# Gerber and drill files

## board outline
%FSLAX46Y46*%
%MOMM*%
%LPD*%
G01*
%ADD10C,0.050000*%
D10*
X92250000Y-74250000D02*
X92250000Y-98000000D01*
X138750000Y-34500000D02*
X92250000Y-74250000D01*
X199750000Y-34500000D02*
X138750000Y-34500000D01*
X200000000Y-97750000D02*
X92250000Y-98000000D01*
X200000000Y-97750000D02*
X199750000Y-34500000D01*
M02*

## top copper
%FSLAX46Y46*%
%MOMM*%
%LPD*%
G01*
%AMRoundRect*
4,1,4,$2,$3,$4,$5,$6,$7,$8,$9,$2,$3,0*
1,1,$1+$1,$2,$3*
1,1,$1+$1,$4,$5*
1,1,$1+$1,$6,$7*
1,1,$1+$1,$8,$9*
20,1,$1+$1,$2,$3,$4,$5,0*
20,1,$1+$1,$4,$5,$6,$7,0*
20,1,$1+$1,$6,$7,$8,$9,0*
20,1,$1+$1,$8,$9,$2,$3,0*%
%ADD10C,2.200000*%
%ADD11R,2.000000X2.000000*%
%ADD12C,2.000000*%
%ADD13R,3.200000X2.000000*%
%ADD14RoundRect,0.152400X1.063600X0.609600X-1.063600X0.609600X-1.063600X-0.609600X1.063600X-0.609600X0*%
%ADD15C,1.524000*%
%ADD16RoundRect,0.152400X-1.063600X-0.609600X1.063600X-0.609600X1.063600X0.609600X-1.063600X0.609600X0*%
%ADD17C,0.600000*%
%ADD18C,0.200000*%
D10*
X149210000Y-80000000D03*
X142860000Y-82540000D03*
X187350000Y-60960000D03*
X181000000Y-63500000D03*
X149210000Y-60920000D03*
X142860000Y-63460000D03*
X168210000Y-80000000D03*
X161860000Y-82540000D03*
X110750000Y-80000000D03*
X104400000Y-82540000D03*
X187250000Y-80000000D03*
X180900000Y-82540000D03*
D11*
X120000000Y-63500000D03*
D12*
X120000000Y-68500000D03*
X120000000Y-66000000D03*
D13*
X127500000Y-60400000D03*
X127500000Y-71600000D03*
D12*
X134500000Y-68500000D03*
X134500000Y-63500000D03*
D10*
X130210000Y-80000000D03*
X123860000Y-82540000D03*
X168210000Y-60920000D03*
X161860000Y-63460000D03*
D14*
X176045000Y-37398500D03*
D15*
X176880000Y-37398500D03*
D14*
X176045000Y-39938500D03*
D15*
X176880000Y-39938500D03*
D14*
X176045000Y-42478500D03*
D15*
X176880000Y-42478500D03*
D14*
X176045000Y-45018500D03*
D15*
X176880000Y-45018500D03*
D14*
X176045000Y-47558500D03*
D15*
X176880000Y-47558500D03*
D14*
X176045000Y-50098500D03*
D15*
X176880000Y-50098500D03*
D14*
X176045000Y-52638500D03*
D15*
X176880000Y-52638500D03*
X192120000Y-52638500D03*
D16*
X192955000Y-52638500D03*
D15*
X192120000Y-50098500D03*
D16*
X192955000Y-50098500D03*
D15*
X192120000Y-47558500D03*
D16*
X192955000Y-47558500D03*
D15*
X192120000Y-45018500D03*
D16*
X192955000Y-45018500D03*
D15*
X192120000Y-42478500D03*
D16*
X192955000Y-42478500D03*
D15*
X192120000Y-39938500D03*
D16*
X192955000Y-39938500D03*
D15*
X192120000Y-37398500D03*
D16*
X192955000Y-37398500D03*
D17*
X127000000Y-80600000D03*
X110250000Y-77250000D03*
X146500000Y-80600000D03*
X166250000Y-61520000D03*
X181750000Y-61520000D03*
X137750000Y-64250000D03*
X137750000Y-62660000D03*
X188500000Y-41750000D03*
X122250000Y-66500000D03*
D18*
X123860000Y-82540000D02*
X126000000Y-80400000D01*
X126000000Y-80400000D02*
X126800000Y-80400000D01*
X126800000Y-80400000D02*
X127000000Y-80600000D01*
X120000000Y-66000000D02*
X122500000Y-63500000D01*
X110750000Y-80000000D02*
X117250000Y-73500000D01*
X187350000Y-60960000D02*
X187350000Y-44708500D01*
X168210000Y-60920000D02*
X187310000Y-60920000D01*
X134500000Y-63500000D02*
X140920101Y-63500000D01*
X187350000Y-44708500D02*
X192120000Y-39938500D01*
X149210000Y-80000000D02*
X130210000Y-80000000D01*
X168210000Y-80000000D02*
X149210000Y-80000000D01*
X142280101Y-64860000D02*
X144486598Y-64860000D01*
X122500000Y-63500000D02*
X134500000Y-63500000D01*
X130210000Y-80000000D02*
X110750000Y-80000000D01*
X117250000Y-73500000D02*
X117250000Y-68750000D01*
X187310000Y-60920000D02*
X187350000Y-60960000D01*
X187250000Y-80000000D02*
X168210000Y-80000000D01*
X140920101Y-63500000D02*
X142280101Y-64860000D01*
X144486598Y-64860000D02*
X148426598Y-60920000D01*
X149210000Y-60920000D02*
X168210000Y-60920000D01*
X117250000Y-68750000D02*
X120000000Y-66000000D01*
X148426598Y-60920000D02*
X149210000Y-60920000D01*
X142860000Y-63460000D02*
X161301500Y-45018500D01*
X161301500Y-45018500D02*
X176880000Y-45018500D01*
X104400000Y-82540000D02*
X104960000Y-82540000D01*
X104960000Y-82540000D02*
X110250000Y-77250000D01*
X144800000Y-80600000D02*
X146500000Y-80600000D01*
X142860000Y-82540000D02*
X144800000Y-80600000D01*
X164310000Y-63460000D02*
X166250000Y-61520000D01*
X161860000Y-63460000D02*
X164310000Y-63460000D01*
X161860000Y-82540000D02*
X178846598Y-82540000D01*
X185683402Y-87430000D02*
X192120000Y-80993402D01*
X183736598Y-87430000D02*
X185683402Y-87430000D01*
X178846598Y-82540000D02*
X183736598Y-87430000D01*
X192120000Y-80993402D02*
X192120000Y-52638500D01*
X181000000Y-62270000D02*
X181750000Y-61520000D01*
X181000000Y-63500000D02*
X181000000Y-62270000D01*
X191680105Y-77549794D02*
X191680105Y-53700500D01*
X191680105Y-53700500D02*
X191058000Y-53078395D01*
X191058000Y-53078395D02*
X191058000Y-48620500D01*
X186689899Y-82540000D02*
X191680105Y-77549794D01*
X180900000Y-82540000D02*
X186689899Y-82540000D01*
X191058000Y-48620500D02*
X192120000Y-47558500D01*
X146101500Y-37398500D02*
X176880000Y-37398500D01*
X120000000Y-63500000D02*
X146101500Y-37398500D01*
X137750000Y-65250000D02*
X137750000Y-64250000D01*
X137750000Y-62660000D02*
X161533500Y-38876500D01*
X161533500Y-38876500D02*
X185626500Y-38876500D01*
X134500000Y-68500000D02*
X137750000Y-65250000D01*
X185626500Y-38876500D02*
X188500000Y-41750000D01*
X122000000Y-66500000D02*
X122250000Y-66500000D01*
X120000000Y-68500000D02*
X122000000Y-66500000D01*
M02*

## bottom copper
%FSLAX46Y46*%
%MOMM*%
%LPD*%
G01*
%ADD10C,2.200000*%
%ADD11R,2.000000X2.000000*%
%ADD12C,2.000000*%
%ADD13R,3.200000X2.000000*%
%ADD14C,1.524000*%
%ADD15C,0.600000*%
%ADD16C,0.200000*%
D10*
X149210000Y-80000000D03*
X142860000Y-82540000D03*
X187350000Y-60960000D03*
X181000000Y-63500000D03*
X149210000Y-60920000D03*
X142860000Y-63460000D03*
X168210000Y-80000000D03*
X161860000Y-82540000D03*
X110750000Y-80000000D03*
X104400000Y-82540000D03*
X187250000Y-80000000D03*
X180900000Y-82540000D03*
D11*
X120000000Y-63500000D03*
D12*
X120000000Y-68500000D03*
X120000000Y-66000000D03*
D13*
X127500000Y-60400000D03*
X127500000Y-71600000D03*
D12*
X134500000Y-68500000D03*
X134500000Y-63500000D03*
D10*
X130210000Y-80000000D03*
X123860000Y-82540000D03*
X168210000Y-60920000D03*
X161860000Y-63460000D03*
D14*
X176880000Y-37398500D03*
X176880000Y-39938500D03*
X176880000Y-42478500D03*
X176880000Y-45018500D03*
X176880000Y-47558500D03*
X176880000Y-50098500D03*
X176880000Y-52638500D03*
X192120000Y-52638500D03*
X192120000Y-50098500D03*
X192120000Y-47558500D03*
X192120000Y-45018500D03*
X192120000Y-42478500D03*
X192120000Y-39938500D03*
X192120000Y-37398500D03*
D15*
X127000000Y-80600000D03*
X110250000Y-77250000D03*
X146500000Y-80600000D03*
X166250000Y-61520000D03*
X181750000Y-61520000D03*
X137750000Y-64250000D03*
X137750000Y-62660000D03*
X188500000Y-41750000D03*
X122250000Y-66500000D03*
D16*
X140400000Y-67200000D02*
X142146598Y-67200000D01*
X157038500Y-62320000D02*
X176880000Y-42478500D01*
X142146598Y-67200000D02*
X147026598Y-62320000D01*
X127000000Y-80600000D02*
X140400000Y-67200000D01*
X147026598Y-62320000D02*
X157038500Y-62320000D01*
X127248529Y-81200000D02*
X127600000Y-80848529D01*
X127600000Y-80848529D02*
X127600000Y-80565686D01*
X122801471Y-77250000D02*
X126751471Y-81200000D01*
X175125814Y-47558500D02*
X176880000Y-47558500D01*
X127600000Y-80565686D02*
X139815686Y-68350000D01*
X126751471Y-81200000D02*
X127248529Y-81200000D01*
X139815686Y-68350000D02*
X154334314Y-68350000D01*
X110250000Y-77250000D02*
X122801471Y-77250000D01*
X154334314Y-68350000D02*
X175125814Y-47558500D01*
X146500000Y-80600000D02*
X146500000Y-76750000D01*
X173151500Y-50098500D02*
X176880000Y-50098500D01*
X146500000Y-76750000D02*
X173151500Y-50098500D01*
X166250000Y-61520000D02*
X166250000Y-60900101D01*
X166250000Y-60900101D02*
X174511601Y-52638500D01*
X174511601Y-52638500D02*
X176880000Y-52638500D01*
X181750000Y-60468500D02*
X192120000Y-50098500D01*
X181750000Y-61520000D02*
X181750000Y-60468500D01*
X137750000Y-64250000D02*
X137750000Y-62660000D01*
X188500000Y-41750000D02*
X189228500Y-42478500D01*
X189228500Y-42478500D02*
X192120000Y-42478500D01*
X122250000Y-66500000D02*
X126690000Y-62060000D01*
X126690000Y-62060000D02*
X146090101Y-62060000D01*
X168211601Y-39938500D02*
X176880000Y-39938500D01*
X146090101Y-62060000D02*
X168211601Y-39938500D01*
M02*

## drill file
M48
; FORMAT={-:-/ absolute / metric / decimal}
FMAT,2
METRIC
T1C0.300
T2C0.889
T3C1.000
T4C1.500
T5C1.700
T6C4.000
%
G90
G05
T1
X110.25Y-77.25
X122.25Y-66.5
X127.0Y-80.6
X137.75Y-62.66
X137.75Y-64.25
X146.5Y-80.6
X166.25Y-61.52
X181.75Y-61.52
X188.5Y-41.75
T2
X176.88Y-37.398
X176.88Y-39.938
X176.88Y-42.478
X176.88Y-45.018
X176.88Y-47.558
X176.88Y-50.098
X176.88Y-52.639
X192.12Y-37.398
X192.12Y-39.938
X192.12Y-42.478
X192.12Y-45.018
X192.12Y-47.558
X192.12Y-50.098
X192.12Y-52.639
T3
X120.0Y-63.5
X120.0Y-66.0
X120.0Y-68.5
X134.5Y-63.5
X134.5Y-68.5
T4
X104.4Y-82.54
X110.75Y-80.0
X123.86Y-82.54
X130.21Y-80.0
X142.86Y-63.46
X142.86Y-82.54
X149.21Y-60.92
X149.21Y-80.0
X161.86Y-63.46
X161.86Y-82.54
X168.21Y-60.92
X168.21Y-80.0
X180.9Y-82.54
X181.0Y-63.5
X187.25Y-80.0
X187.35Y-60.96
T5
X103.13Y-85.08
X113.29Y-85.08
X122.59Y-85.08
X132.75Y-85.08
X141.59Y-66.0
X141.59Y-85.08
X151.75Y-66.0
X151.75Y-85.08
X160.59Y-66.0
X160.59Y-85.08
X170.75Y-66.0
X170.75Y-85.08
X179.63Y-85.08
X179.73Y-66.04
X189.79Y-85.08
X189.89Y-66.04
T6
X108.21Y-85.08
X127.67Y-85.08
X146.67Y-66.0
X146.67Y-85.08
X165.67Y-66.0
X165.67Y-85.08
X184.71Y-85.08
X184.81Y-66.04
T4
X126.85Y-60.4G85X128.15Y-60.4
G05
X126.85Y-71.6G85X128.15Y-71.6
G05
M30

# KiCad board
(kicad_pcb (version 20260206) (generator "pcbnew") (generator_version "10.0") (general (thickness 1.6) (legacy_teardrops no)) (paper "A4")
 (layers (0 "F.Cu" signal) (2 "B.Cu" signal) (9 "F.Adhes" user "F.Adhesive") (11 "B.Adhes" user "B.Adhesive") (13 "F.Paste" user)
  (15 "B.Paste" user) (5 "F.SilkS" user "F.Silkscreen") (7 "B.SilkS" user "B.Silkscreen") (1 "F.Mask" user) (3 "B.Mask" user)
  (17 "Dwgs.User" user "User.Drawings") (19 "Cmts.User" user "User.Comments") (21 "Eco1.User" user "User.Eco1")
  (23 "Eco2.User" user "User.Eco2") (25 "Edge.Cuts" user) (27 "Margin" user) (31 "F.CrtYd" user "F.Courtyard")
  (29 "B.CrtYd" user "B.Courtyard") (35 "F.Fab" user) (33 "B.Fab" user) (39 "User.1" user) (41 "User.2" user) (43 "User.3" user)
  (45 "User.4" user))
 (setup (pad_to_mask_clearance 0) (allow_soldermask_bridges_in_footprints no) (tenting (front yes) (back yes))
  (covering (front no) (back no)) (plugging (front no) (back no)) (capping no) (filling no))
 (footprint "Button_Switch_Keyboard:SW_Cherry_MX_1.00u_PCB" (layer "F.Cu") (at 149.21 80)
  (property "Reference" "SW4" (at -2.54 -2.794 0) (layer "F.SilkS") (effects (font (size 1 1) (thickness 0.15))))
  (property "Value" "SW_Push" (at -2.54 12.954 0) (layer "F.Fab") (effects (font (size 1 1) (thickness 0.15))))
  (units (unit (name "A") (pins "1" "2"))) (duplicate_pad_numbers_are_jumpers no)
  (pad "" np_thru_hole circle (at -7.62 5.08) (size 1.7 1.7) (drill 1.7) (layers "*.Cu" "*.Mask"))
  (pad "" np_thru_hole circle (at -2.54 5.08) (size 4 4) (drill 4) (layers "*.Cu" "*.Mask"))
  (pad "" np_thru_hole circle (at 2.54 5.08) (size 1.7 1.7) (drill 1.7) (layers "*.Cu" "*.Mask"))
  (pad "1" thru_hole circle (at 0 0) (size 2.2 2.2) (drill 1.5) (layers "*.Cu" "*.Mask") (remove_unused_layers no) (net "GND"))
  (pad "2" thru_hole circle (at -6.35 2.54) (size 2.2 2.2) (drill 1.5) (layers "*.Cu" "*.Mask") (remove_unused_layers no)
   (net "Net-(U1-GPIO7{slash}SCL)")))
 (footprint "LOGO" (layer "F.Cu") (at 117.485008 73.126205 90)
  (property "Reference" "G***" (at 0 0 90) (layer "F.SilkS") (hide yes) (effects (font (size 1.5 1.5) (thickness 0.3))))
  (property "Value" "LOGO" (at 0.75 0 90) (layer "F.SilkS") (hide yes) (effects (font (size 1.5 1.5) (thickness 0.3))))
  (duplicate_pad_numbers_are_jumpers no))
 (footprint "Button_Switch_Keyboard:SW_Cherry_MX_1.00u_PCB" (layer "F.Cu") (at 187.35 60.96)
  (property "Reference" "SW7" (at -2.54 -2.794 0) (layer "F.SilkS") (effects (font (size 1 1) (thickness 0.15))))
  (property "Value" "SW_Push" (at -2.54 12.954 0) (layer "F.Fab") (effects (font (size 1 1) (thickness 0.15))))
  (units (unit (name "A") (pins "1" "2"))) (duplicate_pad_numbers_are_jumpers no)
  (pad "" np_thru_hole circle (at -7.62 5.08) (size 1.7 1.7) (drill 1.7) (layers "*.Cu" "*.Mask"))
  (pad "" np_thru_hole circle (at -2.54 5.08) (size 4 4) (drill 4) (layers "*.Cu" "*.Mask"))
  (pad "" np_thru_hole circle (at 2.54 5.08) (size 1.7 1.7) (drill 1.7) (layers "*.Cu" "*.Mask"))
  (pad "1" thru_hole circle (at 0 0) (size 2.2 2.2) (drill 1.5) (layers "*.Cu" "*.Mask") (remove_unused_layers no) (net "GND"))
  (pad "2" thru_hole circle (at -6.35 2.54) (size 2.2 2.2) (drill 1.5) (layers "*.Cu" "*.Mask") (remove_unused_layers no)
   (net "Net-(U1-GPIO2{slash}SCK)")))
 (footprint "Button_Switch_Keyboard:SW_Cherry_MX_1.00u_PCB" (layer "F.Cu") (at 149.21 60.92)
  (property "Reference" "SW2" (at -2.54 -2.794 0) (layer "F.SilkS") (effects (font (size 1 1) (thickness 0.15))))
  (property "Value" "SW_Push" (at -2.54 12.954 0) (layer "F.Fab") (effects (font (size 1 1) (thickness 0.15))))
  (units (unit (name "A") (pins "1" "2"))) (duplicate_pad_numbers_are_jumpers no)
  (pad "" np_thru_hole circle (at -7.62 5.08) (size 1.7 1.7) (drill 1.7) (layers "*.Cu" "*.Mask"))
  (pad "" np_thru_hole circle (at -2.54 5.08) (size 4 4) (drill 4) (layers "*.Cu" "*.Mask"))
  (pad "" np_thru_hole circle (at 2.54 5.08) (size 1.7 1.7) (drill 1.7) (layers "*.Cu" "*.Mask"))
  (pad "1" thru_hole circle (at 0 0) (size 2.2 2.2) (drill 1.5) (layers "*.Cu" "*.Mask") (remove_unused_layers no) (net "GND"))
  (pad "2" thru_hole circle (at -6.35 2.54) (size 2.2 2.2) (drill 1.5) (layers "*.Cu" "*.Mask") (remove_unused_layers no)
   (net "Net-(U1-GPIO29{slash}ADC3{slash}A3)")))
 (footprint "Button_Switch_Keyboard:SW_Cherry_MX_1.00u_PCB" (layer "F.Cu") (at 168.21 80)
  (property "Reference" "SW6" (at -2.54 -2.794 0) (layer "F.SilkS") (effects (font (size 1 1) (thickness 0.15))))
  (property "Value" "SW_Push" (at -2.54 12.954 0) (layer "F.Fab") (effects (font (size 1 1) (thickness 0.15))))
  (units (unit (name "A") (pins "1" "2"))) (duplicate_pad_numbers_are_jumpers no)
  (pad "" np_thru_hole circle (at -7.62 5.08) (size 1.7 1.7) (drill 1.7) (layers "*.Cu" "*.Mask"))
  (pad "" np_thru_hole circle (at -2.54 5.08) (size 4 4) (drill 4) (layers "*.Cu" "*.Mask"))
  (pad "" np_thru_hole circle (at 2.54 5.08) (size 1.7 1.7) (drill 1.7) (layers "*.Cu" "*.Mask"))
  (pad "1" thru_hole circle (at 0 0) (size 2.2 2.2) (drill 1.5) (layers "*.Cu" "*.Mask") (remove_unused_layers no) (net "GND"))
  (pad "2" thru_hole circle (at -6.35 2.54) (size 2.2 2.2) (drill 1.5) (layers "*.Cu" "*.Mask") (remove_unused_layers no)
   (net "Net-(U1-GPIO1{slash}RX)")))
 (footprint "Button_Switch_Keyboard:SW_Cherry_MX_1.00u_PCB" (layer "F.Cu") (at 110.75 80)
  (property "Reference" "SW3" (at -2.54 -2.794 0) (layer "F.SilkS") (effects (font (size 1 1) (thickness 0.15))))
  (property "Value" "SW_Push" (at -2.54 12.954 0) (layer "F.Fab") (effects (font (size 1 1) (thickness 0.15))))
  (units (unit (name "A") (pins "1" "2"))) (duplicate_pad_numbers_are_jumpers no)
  (pad "" np_thru_hole circle (at -7.62 5.08) (size 1.7 1.7) (drill 1.7) (layers "*.Cu" "*.Mask"))
  (pad "" np_thru_hole circle (at -2.54 5.08) (size 4 4) (drill 4) (layers "*.Cu" "*.Mask"))
  (pad "" np_thru_hole circle (at 2.54 5.08) (size 1.7 1.7) (drill 1.7) (layers "*.Cu" "*.Mask"))
  (pad "1" thru_hole circle (at 0 0) (size 2.2 2.2) (drill 1.5) (layers "*.Cu" "*.Mask") (remove_unused_layers no) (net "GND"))
  (pad "2" thru_hole circle (at -6.35 2.54) (size 2.2 2.2) (drill 1.5) (layers "*.Cu" "*.Mask") (remove_unused_layers no)
   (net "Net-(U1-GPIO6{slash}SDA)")))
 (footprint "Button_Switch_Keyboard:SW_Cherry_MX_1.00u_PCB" (layer "F.Cu") (at 187.25 80)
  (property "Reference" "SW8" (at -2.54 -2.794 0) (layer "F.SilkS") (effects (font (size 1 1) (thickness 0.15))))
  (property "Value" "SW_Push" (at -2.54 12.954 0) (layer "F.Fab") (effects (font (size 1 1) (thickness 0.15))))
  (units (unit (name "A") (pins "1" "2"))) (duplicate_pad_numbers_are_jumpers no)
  (pad "" np_thru_hole circle (at -7.62 5.08) (size 1.7 1.7) (drill 1.7) (layers "*.Cu" "*.Mask"))
  (pad "" np_thru_hole circle (at -2.54 5.08) (size 4 4) (drill 4) (layers "*.Cu" "*.Mask"))
  (pad "" np_thru_hole circle (at 2.54 5.08) (size 1.7 1.7) (drill 1.7) (layers "*.Cu" "*.Mask"))
  (pad "1" thru_hole circle (at 0 0) (size 2.2 2.2) (drill 1.5) (layers "*.Cu" "*.Mask") (remove_unused_layers no) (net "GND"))
  (pad "2" thru_hole circle (at -6.35 2.54) (size 2.2 2.2) (drill 1.5) (layers "*.Cu" "*.Mask") (remove_unused_layers no)
   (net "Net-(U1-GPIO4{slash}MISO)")))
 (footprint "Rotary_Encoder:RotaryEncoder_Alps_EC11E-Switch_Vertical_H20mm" (layer "F.Cu") (at 120 63.5)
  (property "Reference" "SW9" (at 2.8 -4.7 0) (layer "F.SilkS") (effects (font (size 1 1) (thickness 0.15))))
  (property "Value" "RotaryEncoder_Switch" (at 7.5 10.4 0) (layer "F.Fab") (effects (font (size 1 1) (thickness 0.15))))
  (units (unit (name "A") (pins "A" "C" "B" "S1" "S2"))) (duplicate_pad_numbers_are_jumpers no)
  (pad "A" thru_hole rect (at 0 0) (size 2 2) (drill 1) (layers "*.Cu" "*.Mask") (remove_unused_layers no)
   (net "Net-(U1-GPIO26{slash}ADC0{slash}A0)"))
  (pad "B" thru_hole circle (at 0 5) (size 2 2) (drill 1) (layers "*.Cu" "*.Mask") (remove_unused_layers no)
   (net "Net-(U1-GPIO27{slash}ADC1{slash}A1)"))
  (pad "C" thru_hole circle (at 0 2.5) (size 2 2) (drill 1) (layers "*.Cu" "*.Mask") (remove_unused_layers no) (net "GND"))
  (pad "MP" thru_hole rect (at 7.5 -3.1) (size 3.2 2) (drill oval 2.8 1.5) (layers "*.Cu" "*.Mask") (remove_unused_layers no))
  (pad "MP" thru_hole rect (at 7.5 8.1) (size 3.2 2) (drill oval 2.8 1.5) (layers "*.Cu" "*.Mask") (remove_unused_layers no))
  (pad "S1" thru_hole circle (at 14.5 5) (size 2 2) (drill 1) (layers "*.Cu" "*.Mask") (remove_unused_layers no) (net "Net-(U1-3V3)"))
  (pad "S2" thru_hole circle (at 14.5 0) (size 2 2) (drill 1) (layers "*.Cu" "*.Mask") (remove_unused_layers no) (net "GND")))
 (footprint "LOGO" (layer "F.Cu") (at 167.351488 86.633252)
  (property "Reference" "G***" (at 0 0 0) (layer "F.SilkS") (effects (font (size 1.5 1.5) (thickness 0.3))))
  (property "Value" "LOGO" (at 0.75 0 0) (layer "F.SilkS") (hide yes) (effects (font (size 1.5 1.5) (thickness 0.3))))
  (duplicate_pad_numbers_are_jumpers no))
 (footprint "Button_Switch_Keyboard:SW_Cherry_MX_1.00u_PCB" (layer "F.Cu") (at 130.21 80)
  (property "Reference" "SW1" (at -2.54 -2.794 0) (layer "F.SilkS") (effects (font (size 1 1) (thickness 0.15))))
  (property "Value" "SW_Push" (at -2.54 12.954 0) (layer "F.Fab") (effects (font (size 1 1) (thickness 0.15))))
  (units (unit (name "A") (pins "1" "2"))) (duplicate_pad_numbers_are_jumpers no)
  (pad "" np_thru_hole circle (at -7.62 5.08) (size 1.7 1.7) (drill 1.7) (layers "*.Cu" "*.Mask"))
  (pad "" np_thru_hole circle (at -2.54 5.08) (size 4 4) (drill 4) (layers "*.Cu" "*.Mask"))
  (pad "" np_thru_hole circle (at 2.54 5.08) (size 1.7 1.7) (drill 1.7) (layers "*.Cu" "*.Mask"))
  (pad "1" thru_hole circle (at 0 0) (size 2.2 2.2) (drill 1.5) (layers "*.Cu" "*.Mask") (remove_unused_layers no) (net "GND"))
  (pad "2" thru_hole circle (at -6.35 2.54) (size 2.2 2.2) (drill 1.5) (layers "*.Cu" "*.Mask") (remove_unused_layers no)
   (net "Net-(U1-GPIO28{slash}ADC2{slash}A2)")))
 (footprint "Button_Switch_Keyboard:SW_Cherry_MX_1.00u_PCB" (layer "F.Cu") (at 168.21 60.92)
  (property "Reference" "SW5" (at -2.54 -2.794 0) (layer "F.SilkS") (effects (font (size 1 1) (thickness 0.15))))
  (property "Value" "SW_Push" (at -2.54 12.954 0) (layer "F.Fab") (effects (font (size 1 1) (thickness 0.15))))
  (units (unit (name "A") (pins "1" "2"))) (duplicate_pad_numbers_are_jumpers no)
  (pad "" np_thru_hole circle (at -7.62 5.08) (size 1.7 1.7) (drill 1.7) (layers "*.Cu" "*.Mask"))
  (pad "" np_thru_hole circle (at -2.54 5.08) (size 4 4) (drill 4) (layers "*.Cu" "*.Mask"))
  (pad "" np_thru_hole circle (at 2.54 5.08) (size 1.7 1.7) (drill 1.7) (layers "*.Cu" "*.Mask"))
  (pad "1" thru_hole circle (at 0 0) (size 2.2 2.2) (drill 1.5) (layers "*.Cu" "*.Mask") (remove_unused_layers no) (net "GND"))
  (pad "2" thru_hole circle (at -6.35 2.54) (size 2.2 2.2) (drill 1.5) (layers "*.Cu" "*.Mask") (remove_unused_layers no)
   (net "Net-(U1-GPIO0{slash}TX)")))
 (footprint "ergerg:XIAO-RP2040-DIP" (layer "F.Cu") (at 184.5 45.0185)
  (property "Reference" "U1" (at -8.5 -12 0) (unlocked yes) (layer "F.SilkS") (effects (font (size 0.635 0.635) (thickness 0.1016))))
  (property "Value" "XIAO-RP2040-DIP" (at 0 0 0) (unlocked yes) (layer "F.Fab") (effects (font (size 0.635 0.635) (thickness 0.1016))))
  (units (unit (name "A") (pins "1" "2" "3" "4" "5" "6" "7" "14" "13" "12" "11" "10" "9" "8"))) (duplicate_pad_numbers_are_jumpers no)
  (pad "1" smd roundrect (at -8.455 -7.62 180) (size 2.432 1.524) (layers "F.Cu" "F.Mask") (roundrect_rratio 0.1)
   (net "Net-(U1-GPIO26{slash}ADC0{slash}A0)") (thermal_bridge_angle 45))
  (pad "1" thru_hole circle (at -7.62 -7.62 180) (size 1.524 1.524) (drill 0.889) (layers "*.Cu" "*.Mask") (remove_unused_layers no)
   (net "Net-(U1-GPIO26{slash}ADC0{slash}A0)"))
  (pad "2" smd roundrect (at -8.455 -5.08 180) (size 2.432 1.524) (layers "F.Cu" "F.Mask") (roundrect_rratio 0.1)
   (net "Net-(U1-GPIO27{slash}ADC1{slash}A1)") (thermal_bridge_angle 45))
  (pad "2" thru_hole circle (at -7.62 -5.08 180) (size 1.524 1.524) (drill 0.889) (layers "*.Cu" "*.Mask") (remove_unused_layers no)
   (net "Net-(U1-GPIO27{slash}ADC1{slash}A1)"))
  (pad "3" smd roundrect (at -8.455 -2.54 180) (size 2.432 1.524) (layers "F.Cu" "F.Mask") (roundrect_rratio 0.1)
   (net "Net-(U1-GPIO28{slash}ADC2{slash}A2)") (thermal_bridge_angle 45))
  (pad "3" thru_hole circle (at -7.62 -2.54 180) (size 1.524 1.524) (drill 0.889) (layers "*.Cu" "*.Mask") (remove_unused_layers no)
   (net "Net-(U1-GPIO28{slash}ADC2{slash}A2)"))
  (pad "4" smd roundrect (at -8.455 0 180) (size 2.432 1.524) (layers "F.Cu" "F.Mask") (roundrect_rratio 0.1)
   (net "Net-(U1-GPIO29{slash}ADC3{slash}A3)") (thermal_bridge_angle 45))
  (pad "4" thru_hole circle (at -7.62 0 180) (size 1.524 1.524) (drill 0.889) (layers "*.Cu" "*.Mask") (remove_unused_layers no)
   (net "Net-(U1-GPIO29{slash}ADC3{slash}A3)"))
  (pad "5" smd roundrect (at -8.455 2.54 180) (size 2.432 1.524) (layers "F.Cu" "F.Mask") (roundrect_rratio 0.1)
   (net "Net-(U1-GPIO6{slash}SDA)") (thermal_bridge_angle 45))
  (pad "5" thru_hole circle (at -7.62 2.54 180) (size 1.524 1.524) (drill 0.889) (layers "*.Cu" "*.Mask") (remove_unused_layers no)
   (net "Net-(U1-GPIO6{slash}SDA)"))
  (pad "6" smd roundrect (at -8.455 5.08 180) (size 2.432 1.524) (layers "F.Cu" "F.Mask") (roundrect_rratio 0.1)
   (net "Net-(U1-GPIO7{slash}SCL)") (thermal_bridge_angle 45))
  (pad "6" thru_hole circle (at -7.62 5.08 180) (size 1.524 1.524) (drill 0.889) (layers "*.Cu" "*.Mask") (remove_unused_layers no)
   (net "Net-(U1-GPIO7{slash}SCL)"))
  (pad "7" smd roundrect (at -8.455 7.62 180) (size 2.432 1.524) (layers "F.Cu" "F.Mask") (roundrect_rratio 0.1)
   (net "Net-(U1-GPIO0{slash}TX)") (thermal_bridge_angle 45))
  (pad "7" thru_hole circle (at -7.62 7.62 180) (size 1.524 1.524) (drill 0.889) (layers "*.Cu" "*.Mask") (remove_unused_layers no)
   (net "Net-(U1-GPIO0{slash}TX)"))
  (pad "8" thru_hole circle (at 7.62 7.62) (size 1.524 1.524) (drill 0.889) (layers "*.Cu" "*.Mask") (remove_unused_layers no)
   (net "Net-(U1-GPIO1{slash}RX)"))
  (pad "8" smd roundrect (at 8.455 7.62) (size 2.432 1.524) (layers "F.Cu" "F.Mask") (roundrect_rratio 0.1) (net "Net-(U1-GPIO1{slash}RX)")
   (thermal_bridge_angle 45))
  (pad "9" thru_hole circle (at 7.62 5.08) (size 1.524 1.524) (drill 0.889) (layers "*.Cu" "*.Mask") (remove_unused_layers no)
   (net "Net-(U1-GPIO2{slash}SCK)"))
  (pad "9" smd roundrect (at 8.455 5.08) (size 2.432 1.524) (layers "F.Cu" "F.Mask") (roundrect_rratio 0.1) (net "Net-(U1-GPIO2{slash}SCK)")
   (thermal_bridge_angle 45))
  (pad "10" thru_hole circle (at 7.62 2.54) (size 1.524 1.524) (drill 0.889) (layers "*.Cu" "*.Mask") (remove_unused_layers no)
   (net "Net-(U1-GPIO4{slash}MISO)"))
  (pad "10" smd roundrect (at 8.455 2.54) (size 2.432 1.524) (layers "F.Cu" "F.Mask") (roundrect_rratio 0.1)
   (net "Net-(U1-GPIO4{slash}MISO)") (thermal_bridge_angle 45))
  (pad "11" thru_hole circle (at 7.62 0) (size 1.524 1.524) (drill 0.889) (layers "*.Cu" "*.Mask") (remove_unused_layers no)
   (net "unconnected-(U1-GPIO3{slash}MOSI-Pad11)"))
  (pad "11" smd roundrect (at 8.455 0) (size 2.432 1.524) (layers "F.Cu" "F.Mask") (roundrect_rratio 0.1)
   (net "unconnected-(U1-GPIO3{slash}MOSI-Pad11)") (thermal_bridge_angle 45))
  (pad "12" thru_hole circle (at 7.62 -2.54) (size 1.524 1.524) (drill 0.889) (layers "*.Cu" "*.Mask") (remove_unused_layers no)
   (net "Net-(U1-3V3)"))
  (pad "12" smd roundrect (at 8.455 -2.54) (size 2.432 1.524) (layers "F.Cu" "F.Mask") (roundrect_rratio 0.1) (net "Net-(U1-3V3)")
   (thermal_bridge_angle 45))
  (pad "13" thru_hole circle (at 7.62 -5.08) (size 1.524 1.524) (drill 0.889) (layers "*.Cu" "*.Mask") (remove_unused_layers no) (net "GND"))
  (pad "13" smd roundrect (at 8.455 -5.08) (size 2.432 1.524) (layers "F.Cu" "F.Mask") (roundrect_rratio 0.1) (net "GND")
   (thermal_bridge_angle 45))
  (pad "14" thru_hole circle (at 7.62 -7.62) (size 1.524 1.524) (drill 0.889) (layers "*.Cu" "*.Mask") (remove_unused_layers no) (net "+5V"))
  (pad "14" smd roundrect (at 8.455 -7.62) (size 2.432 1.524) (layers "F.Cu" "F.Mask") (roundrect_rratio 0.1) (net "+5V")
   (thermal_bridge_angle 45)))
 (gr_line (start 92.25 74.25) (end 92.25 98) (stroke (width 0.05) (type default)) (layer "Edge.Cuts"))
 (gr_line (start 138.75 34.5) (end 92.25 74.25) (stroke (width 0.05) (type default)) (layer "Edge.Cuts"))
 (gr_line (start 199.75 34.5) (end 138.75 34.5) (stroke (width 0.05) (type default)) (layer "Edge.Cuts"))
 (gr_line (start 200 97.75) (end 92.25 98) (stroke (width 0.05) (type default)) (layer "Edge.Cuts"))
 (gr_line (start 200 97.75) (end 199.75 34.5) (stroke (width 0.05) (type default)) (layer "Edge.Cuts"))
 (segment (start 123.86 82.54) (end 126 80.4) (width 0.2) (layer "F.Cu") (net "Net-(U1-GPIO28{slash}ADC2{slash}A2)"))
 (segment (start 126 80.4) (end 126.8 80.4) (width 0.2) (layer "F.Cu") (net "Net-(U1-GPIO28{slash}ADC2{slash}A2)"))
 (segment (start 126.8 80.4) (end 127 80.6) (width 0.2) (layer "F.Cu") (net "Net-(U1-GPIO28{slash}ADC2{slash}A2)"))
 (via (at 127 80.6) (size 0.6) (drill 0.3) (layers "F.Cu" "B.Cu") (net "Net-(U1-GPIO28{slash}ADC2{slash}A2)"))
 (segment (start 140.4 67.2) (end 142.146598 67.2) (width 0.2) (layer "B.Cu") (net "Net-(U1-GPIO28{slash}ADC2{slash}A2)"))
 (segment (start 157.0385 62.32) (end 176.88 42.4785) (width 0.2) (layer "B.Cu") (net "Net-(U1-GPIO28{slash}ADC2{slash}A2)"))
 (segment (start 142.146598 67.2) (end 147.026598 62.32) (width 0.2) (layer "B.Cu") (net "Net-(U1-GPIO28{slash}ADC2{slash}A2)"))
 (segment (start 127 80.6) (end 140.4 67.2) (width 0.2) (layer "B.Cu") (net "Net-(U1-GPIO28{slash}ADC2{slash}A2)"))
 (segment (start 147.026598 62.32) (end 157.0385 62.32) (width 0.2) (layer "B.Cu") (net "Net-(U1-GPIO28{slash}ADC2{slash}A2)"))
 (segment (start 120 66) (end 122.5 63.5) (width 0.2) (layer "F.Cu") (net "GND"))
 (segment (start 110.75 80) (end 117.25 73.5) (width 0.2) (layer "F.Cu") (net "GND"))
 (segment (start 187.35 60.96) (end 187.35 44.7085) (width 0.2) (layer "F.Cu") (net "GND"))
 (segment (start 168.21 60.92) (end 187.31 60.92) (width 0.2) (layer "F.Cu") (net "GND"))
 (segment (start 134.5 63.5) (end 140.920101 63.5) (width 0.2) (layer "F.Cu") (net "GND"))
 (segment (start 187.35 44.7085) (end 192.12 39.9385) (width 0.2) (layer "F.Cu") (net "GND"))
 (segment (start 149.21 80) (end 130.21 80) (width 0.2) (layer "F.Cu") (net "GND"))
 (segment (start 168.21 80) (end 149.21 80) (width 0.2) (layer "F.Cu") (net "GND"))
 (segment (start 142.280101 64.86) (end 144.486598 64.86) (width 0.2) (layer "F.Cu") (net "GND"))
 (segment (start 122.5 63.5) (end 134.5 63.5) (width 0.2) (layer "F.Cu") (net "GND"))
 (segment (start 130.21 80) (end 110.75 80) (width 0.2) (layer "F.Cu") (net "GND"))
 (segment (start 117.25 73.5) (end 117.25 68.75) (width 0.2) (layer "F.Cu") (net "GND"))
 (segment (start 187.31 60.92) (end 187.35 60.96) (width 0.2) (layer "F.Cu") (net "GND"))
 (segment (start 187.25 80) (end 168.21 80) (width 0.2) (layer "F.Cu") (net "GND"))
 (segment (start 140.920101 63.5) (end 142.280101 64.86) (width 0.2) (layer "F.Cu") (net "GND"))
 (segment (start 144.486598 64.86) (end 148.426598 60.92) (width 0.2) (layer "F.Cu") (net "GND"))
 (segment (start 149.21 60.92) (end 168.21 60.92) (width 0.2) (layer "F.Cu") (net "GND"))
 (segment (start 117.25 68.75) (end 120 66) (width 0.2) (layer "F.Cu") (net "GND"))
 (segment (start 148.426598 60.92) (end 149.21 60.92) (width 0.2) (layer "F.Cu") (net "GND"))
 (segment (start 142.86 63.46) (end 161.3015 45.0185) (width 0.2) (layer "F.Cu") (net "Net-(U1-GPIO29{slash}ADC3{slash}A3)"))
 (segment (start 161.3015 45.0185) (end 176.88 45.0185) (width 0.2) (layer "F.Cu") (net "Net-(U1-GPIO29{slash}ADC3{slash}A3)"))
 (segment (start 104.4 82.54) (end 104.96 82.54) (width 0.2) (layer "F.Cu") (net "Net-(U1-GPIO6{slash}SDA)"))
 (segment (start 104.96 82.54) (end 110.25 77.25) (width 0.2) (layer "F.Cu") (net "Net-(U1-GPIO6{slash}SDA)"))
 (via (at 110.25 77.25) (size 0.6) (drill 0.3) (layers "F.Cu" "B.Cu") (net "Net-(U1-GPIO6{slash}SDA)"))
 (segment (start 127.248529 81.2) (end 127.6 80.848529) (width 0.2) (layer "B.Cu") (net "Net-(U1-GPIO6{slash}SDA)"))
 (segment (start 127.6 80.848529) (end 127.6 80.565686) (width 0.2) (layer "B.Cu") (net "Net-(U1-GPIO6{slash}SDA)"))
 (segment (start 122.801471 77.25) (end 126.751471 81.2) (width 0.2) (layer "B.Cu") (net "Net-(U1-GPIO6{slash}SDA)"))
 (segment (start 175.125814 47.5585) (end 176.88 47.5585) (width 0.2) (layer "B.Cu") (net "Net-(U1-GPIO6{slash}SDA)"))
 (segment (start 127.6 80.565686) (end 139.815686 68.35) (width 0.2) (layer "B.Cu") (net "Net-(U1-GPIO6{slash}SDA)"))
 (segment (start 126.751471 81.2) (end 127.248529 81.2) (width 0.2) (layer "B.Cu") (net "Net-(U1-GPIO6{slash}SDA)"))
 (segment (start 139.815686 68.35) (end 154.334314 68.35) (width 0.2) (layer "B.Cu") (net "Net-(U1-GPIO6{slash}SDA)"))
 (segment (start 110.25 77.25) (end 122.801471 77.25) (width 0.2) (layer "B.Cu") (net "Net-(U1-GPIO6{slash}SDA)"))
 (segment (start 154.334314 68.35) (end 175.125814 47.5585) (width 0.2) (layer "B.Cu") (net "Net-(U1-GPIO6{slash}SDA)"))
 (segment (start 144.8 80.6) (end 146.5 80.6) (width 0.2) (layer "F.Cu") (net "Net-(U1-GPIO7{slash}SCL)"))
 (segment (start 142.86 82.54) (end 144.8 80.6) (width 0.2) (layer "F.Cu") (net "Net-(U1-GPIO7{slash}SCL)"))
 (via (at 146.5 80.6) (size 0.6) (drill 0.3) (layers "F.Cu" "B.Cu") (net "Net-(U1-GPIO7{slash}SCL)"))
 (segment (start 146.5 80.6) (end 146.5 76.75) (width 0.2) (layer "B.Cu") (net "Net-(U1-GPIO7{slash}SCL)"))
 (segment (start 173.1515 50.0985) (end 176.88 50.0985) (width 0.2) (layer "B.Cu") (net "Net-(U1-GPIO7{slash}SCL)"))
 (segment (start 146.5 76.75) (end 173.1515 50.0985) (width 0.2) (layer "B.Cu") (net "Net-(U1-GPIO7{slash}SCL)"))
 (segment (start 164.31 63.46) (end 166.25 61.52) (width 0.2) (layer "F.Cu") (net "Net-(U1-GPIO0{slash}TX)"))
 (segment (start 161.86 63.46) (end 164.31 63.46) (width 0.2) (layer "F.Cu") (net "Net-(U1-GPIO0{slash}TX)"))
 (via (at 166.25 61.52) (size 0.6) (drill 0.3) (layers "F.Cu" "B.Cu") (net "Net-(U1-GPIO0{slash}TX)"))
 (segment (start 166.25 61.52) (end 166.25 60.900101) (width 0.2) (layer "B.Cu") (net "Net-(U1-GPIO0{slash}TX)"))
 (segment (start 166.25 60.900101) (end 174.511601 52.6385) (width 0.2) (layer "B.Cu") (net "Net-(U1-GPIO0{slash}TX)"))
 (segment (start 174.511601 52.6385) (end 176.88 52.6385) (width 0.2) (layer "B.Cu") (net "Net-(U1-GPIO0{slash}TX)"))
 (segment (start 161.86 82.54) (end 178.846598 82.54) (width 0.2) (layer "F.Cu") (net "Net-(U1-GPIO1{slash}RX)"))
 (segment (start 185.683402 87.43) (end 192.12 80.993402) (width 0.2) (layer "F.Cu") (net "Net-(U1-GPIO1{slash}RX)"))
 (segment (start 183.736598 87.43) (end 185.683402 87.43) (width 0.2) (layer "F.Cu") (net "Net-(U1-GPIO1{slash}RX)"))
 (segment (start 178.846598 82.54) (end 183.736598 87.43) (width 0.2) (layer "F.Cu") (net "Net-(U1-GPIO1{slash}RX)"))
 (segment (start 192.12 80.993402) (end 192.12 52.6385) (width 0.2) (layer "F.Cu") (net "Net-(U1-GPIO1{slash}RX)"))
 (segment (start 181 62.27) (end 181.75 61.52) (width 0.2) (layer "F.Cu") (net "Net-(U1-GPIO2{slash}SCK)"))
 (segment (start 181 63.5) (end 181 62.27) (width 0.2) (layer "F.Cu") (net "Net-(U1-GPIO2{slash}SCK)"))
 (via (at 181.75 61.52) (size 0.6) (drill 0.3) (layers "F.Cu" "B.Cu") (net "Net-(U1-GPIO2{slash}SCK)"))
 (segment (start 181.75 60.4685) (end 192.12 50.0985) (width 0.2) (layer "B.Cu") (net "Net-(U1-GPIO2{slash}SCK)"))
 (segment (start 181.75 61.52) (end 181.75 60.4685) (width 0.2) (layer "B.Cu") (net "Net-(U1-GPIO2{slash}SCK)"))
 (segment (start 191.680105 77.549794) (end 191.680105 53.7005) (width 0.2) (layer "F.Cu") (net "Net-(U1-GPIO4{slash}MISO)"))
 (segment (start 191.680105 53.7005) (end 191.058 53.078395) (width 0.2) (layer "F.Cu") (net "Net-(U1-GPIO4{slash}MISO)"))
 (segment (start 191.058 53.078395) (end 191.058 48.6205) (width 0.2) (layer "F.Cu") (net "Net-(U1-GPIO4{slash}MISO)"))
 (segment (start 186.689899 82.54) (end 191.680105 77.549794) (width 0.2) (layer "F.Cu") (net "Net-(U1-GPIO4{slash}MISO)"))
 (segment (start 180.9 82.54) (end 186.689899 82.54) (width 0.2) (layer "F.Cu") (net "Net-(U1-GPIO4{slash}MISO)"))
 (segment (start 191.058 48.6205) (end 192.12 47.5585) (width 0.2) (layer "F.Cu") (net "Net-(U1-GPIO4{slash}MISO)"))
 (segment (start 146.1015 37.3985) (end 176.88 37.3985) (width 0.2) (layer "F.Cu") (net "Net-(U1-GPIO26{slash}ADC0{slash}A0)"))
 (segment (start 120 63.5) (end 146.1015 37.3985) (width 0.2) (layer "F.Cu") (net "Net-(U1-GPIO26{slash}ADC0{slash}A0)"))
 (segment (start 137.75 65.25) (end 137.75 64.25) (width 0.2) (layer "F.Cu") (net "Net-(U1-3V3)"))
 (segment (start 137.75 62.66) (end 161.5335 38.8765) (width 0.2) (layer "F.Cu") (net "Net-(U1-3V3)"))
 (segment (start 161.5335 38.8765) (end 185.6265 38.8765) (width 0.2) (layer "F.Cu") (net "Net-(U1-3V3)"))
 (segment (start 134.5 68.5) (end 137.75 65.25) (width 0.2) (layer "F.Cu") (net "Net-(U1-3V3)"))
 (segment (start 185.6265 38.8765) (end 188.5 41.75) (width 0.2) (layer "F.Cu") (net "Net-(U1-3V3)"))
 (via (at 137.75 64.25) (size 0.6) (drill 0.3) (layers "F.Cu" "B.Cu") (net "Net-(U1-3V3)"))
 (via (at 137.75 62.66) (size 0.6) (drill 0.3) (layers "F.Cu" "B.Cu") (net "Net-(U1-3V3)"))
 (via (at 188.5 41.75) (size 0.6) (drill 0.3) (layers "F.Cu" "B.Cu") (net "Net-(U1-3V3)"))
 (segment (start 137.75 64.25) (end 137.75 62.66) (width 0.2) (layer "B.Cu") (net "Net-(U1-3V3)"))
 (segment (start 188.5 41.75) (end 189.2285 42.4785) (width 0.2) (layer "B.Cu") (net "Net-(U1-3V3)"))
 (segment (start 189.2285 42.4785) (end 192.12 42.4785) (width 0.2) (layer "B.Cu") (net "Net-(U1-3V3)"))
 (segment (start 122 66.5) (end 122.25 66.5) (width 0.2) (layer "F.Cu") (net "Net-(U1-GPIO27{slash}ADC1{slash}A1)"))
 (segment (start 120 68.5) (end 122 66.5) (width 0.2) (layer "F.Cu") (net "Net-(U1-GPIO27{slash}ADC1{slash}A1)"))
 (via (at 122.25 66.5) (size 0.6) (drill 0.3) (layers "F.Cu" "B.Cu") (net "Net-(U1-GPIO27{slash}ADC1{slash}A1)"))
 (segment (start 122.25 66.5) (end 126.69 62.06) (width 0.2) (layer "B.Cu") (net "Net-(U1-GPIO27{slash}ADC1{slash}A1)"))
 (segment (start 126.69 62.06) (end 146.090101 62.06) (width 0.2) (layer "B.Cu") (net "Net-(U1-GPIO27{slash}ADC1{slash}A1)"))
 (segment (start 168.211601 39.9385) (end 176.88 39.9385) (width 0.2) (layer "B.Cu") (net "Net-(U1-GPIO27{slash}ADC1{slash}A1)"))
 (segment (start 146.090101 62.06) (end 168.211601 39.9385) (width 0.2) (layer "B.Cu") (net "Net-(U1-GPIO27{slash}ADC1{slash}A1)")))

